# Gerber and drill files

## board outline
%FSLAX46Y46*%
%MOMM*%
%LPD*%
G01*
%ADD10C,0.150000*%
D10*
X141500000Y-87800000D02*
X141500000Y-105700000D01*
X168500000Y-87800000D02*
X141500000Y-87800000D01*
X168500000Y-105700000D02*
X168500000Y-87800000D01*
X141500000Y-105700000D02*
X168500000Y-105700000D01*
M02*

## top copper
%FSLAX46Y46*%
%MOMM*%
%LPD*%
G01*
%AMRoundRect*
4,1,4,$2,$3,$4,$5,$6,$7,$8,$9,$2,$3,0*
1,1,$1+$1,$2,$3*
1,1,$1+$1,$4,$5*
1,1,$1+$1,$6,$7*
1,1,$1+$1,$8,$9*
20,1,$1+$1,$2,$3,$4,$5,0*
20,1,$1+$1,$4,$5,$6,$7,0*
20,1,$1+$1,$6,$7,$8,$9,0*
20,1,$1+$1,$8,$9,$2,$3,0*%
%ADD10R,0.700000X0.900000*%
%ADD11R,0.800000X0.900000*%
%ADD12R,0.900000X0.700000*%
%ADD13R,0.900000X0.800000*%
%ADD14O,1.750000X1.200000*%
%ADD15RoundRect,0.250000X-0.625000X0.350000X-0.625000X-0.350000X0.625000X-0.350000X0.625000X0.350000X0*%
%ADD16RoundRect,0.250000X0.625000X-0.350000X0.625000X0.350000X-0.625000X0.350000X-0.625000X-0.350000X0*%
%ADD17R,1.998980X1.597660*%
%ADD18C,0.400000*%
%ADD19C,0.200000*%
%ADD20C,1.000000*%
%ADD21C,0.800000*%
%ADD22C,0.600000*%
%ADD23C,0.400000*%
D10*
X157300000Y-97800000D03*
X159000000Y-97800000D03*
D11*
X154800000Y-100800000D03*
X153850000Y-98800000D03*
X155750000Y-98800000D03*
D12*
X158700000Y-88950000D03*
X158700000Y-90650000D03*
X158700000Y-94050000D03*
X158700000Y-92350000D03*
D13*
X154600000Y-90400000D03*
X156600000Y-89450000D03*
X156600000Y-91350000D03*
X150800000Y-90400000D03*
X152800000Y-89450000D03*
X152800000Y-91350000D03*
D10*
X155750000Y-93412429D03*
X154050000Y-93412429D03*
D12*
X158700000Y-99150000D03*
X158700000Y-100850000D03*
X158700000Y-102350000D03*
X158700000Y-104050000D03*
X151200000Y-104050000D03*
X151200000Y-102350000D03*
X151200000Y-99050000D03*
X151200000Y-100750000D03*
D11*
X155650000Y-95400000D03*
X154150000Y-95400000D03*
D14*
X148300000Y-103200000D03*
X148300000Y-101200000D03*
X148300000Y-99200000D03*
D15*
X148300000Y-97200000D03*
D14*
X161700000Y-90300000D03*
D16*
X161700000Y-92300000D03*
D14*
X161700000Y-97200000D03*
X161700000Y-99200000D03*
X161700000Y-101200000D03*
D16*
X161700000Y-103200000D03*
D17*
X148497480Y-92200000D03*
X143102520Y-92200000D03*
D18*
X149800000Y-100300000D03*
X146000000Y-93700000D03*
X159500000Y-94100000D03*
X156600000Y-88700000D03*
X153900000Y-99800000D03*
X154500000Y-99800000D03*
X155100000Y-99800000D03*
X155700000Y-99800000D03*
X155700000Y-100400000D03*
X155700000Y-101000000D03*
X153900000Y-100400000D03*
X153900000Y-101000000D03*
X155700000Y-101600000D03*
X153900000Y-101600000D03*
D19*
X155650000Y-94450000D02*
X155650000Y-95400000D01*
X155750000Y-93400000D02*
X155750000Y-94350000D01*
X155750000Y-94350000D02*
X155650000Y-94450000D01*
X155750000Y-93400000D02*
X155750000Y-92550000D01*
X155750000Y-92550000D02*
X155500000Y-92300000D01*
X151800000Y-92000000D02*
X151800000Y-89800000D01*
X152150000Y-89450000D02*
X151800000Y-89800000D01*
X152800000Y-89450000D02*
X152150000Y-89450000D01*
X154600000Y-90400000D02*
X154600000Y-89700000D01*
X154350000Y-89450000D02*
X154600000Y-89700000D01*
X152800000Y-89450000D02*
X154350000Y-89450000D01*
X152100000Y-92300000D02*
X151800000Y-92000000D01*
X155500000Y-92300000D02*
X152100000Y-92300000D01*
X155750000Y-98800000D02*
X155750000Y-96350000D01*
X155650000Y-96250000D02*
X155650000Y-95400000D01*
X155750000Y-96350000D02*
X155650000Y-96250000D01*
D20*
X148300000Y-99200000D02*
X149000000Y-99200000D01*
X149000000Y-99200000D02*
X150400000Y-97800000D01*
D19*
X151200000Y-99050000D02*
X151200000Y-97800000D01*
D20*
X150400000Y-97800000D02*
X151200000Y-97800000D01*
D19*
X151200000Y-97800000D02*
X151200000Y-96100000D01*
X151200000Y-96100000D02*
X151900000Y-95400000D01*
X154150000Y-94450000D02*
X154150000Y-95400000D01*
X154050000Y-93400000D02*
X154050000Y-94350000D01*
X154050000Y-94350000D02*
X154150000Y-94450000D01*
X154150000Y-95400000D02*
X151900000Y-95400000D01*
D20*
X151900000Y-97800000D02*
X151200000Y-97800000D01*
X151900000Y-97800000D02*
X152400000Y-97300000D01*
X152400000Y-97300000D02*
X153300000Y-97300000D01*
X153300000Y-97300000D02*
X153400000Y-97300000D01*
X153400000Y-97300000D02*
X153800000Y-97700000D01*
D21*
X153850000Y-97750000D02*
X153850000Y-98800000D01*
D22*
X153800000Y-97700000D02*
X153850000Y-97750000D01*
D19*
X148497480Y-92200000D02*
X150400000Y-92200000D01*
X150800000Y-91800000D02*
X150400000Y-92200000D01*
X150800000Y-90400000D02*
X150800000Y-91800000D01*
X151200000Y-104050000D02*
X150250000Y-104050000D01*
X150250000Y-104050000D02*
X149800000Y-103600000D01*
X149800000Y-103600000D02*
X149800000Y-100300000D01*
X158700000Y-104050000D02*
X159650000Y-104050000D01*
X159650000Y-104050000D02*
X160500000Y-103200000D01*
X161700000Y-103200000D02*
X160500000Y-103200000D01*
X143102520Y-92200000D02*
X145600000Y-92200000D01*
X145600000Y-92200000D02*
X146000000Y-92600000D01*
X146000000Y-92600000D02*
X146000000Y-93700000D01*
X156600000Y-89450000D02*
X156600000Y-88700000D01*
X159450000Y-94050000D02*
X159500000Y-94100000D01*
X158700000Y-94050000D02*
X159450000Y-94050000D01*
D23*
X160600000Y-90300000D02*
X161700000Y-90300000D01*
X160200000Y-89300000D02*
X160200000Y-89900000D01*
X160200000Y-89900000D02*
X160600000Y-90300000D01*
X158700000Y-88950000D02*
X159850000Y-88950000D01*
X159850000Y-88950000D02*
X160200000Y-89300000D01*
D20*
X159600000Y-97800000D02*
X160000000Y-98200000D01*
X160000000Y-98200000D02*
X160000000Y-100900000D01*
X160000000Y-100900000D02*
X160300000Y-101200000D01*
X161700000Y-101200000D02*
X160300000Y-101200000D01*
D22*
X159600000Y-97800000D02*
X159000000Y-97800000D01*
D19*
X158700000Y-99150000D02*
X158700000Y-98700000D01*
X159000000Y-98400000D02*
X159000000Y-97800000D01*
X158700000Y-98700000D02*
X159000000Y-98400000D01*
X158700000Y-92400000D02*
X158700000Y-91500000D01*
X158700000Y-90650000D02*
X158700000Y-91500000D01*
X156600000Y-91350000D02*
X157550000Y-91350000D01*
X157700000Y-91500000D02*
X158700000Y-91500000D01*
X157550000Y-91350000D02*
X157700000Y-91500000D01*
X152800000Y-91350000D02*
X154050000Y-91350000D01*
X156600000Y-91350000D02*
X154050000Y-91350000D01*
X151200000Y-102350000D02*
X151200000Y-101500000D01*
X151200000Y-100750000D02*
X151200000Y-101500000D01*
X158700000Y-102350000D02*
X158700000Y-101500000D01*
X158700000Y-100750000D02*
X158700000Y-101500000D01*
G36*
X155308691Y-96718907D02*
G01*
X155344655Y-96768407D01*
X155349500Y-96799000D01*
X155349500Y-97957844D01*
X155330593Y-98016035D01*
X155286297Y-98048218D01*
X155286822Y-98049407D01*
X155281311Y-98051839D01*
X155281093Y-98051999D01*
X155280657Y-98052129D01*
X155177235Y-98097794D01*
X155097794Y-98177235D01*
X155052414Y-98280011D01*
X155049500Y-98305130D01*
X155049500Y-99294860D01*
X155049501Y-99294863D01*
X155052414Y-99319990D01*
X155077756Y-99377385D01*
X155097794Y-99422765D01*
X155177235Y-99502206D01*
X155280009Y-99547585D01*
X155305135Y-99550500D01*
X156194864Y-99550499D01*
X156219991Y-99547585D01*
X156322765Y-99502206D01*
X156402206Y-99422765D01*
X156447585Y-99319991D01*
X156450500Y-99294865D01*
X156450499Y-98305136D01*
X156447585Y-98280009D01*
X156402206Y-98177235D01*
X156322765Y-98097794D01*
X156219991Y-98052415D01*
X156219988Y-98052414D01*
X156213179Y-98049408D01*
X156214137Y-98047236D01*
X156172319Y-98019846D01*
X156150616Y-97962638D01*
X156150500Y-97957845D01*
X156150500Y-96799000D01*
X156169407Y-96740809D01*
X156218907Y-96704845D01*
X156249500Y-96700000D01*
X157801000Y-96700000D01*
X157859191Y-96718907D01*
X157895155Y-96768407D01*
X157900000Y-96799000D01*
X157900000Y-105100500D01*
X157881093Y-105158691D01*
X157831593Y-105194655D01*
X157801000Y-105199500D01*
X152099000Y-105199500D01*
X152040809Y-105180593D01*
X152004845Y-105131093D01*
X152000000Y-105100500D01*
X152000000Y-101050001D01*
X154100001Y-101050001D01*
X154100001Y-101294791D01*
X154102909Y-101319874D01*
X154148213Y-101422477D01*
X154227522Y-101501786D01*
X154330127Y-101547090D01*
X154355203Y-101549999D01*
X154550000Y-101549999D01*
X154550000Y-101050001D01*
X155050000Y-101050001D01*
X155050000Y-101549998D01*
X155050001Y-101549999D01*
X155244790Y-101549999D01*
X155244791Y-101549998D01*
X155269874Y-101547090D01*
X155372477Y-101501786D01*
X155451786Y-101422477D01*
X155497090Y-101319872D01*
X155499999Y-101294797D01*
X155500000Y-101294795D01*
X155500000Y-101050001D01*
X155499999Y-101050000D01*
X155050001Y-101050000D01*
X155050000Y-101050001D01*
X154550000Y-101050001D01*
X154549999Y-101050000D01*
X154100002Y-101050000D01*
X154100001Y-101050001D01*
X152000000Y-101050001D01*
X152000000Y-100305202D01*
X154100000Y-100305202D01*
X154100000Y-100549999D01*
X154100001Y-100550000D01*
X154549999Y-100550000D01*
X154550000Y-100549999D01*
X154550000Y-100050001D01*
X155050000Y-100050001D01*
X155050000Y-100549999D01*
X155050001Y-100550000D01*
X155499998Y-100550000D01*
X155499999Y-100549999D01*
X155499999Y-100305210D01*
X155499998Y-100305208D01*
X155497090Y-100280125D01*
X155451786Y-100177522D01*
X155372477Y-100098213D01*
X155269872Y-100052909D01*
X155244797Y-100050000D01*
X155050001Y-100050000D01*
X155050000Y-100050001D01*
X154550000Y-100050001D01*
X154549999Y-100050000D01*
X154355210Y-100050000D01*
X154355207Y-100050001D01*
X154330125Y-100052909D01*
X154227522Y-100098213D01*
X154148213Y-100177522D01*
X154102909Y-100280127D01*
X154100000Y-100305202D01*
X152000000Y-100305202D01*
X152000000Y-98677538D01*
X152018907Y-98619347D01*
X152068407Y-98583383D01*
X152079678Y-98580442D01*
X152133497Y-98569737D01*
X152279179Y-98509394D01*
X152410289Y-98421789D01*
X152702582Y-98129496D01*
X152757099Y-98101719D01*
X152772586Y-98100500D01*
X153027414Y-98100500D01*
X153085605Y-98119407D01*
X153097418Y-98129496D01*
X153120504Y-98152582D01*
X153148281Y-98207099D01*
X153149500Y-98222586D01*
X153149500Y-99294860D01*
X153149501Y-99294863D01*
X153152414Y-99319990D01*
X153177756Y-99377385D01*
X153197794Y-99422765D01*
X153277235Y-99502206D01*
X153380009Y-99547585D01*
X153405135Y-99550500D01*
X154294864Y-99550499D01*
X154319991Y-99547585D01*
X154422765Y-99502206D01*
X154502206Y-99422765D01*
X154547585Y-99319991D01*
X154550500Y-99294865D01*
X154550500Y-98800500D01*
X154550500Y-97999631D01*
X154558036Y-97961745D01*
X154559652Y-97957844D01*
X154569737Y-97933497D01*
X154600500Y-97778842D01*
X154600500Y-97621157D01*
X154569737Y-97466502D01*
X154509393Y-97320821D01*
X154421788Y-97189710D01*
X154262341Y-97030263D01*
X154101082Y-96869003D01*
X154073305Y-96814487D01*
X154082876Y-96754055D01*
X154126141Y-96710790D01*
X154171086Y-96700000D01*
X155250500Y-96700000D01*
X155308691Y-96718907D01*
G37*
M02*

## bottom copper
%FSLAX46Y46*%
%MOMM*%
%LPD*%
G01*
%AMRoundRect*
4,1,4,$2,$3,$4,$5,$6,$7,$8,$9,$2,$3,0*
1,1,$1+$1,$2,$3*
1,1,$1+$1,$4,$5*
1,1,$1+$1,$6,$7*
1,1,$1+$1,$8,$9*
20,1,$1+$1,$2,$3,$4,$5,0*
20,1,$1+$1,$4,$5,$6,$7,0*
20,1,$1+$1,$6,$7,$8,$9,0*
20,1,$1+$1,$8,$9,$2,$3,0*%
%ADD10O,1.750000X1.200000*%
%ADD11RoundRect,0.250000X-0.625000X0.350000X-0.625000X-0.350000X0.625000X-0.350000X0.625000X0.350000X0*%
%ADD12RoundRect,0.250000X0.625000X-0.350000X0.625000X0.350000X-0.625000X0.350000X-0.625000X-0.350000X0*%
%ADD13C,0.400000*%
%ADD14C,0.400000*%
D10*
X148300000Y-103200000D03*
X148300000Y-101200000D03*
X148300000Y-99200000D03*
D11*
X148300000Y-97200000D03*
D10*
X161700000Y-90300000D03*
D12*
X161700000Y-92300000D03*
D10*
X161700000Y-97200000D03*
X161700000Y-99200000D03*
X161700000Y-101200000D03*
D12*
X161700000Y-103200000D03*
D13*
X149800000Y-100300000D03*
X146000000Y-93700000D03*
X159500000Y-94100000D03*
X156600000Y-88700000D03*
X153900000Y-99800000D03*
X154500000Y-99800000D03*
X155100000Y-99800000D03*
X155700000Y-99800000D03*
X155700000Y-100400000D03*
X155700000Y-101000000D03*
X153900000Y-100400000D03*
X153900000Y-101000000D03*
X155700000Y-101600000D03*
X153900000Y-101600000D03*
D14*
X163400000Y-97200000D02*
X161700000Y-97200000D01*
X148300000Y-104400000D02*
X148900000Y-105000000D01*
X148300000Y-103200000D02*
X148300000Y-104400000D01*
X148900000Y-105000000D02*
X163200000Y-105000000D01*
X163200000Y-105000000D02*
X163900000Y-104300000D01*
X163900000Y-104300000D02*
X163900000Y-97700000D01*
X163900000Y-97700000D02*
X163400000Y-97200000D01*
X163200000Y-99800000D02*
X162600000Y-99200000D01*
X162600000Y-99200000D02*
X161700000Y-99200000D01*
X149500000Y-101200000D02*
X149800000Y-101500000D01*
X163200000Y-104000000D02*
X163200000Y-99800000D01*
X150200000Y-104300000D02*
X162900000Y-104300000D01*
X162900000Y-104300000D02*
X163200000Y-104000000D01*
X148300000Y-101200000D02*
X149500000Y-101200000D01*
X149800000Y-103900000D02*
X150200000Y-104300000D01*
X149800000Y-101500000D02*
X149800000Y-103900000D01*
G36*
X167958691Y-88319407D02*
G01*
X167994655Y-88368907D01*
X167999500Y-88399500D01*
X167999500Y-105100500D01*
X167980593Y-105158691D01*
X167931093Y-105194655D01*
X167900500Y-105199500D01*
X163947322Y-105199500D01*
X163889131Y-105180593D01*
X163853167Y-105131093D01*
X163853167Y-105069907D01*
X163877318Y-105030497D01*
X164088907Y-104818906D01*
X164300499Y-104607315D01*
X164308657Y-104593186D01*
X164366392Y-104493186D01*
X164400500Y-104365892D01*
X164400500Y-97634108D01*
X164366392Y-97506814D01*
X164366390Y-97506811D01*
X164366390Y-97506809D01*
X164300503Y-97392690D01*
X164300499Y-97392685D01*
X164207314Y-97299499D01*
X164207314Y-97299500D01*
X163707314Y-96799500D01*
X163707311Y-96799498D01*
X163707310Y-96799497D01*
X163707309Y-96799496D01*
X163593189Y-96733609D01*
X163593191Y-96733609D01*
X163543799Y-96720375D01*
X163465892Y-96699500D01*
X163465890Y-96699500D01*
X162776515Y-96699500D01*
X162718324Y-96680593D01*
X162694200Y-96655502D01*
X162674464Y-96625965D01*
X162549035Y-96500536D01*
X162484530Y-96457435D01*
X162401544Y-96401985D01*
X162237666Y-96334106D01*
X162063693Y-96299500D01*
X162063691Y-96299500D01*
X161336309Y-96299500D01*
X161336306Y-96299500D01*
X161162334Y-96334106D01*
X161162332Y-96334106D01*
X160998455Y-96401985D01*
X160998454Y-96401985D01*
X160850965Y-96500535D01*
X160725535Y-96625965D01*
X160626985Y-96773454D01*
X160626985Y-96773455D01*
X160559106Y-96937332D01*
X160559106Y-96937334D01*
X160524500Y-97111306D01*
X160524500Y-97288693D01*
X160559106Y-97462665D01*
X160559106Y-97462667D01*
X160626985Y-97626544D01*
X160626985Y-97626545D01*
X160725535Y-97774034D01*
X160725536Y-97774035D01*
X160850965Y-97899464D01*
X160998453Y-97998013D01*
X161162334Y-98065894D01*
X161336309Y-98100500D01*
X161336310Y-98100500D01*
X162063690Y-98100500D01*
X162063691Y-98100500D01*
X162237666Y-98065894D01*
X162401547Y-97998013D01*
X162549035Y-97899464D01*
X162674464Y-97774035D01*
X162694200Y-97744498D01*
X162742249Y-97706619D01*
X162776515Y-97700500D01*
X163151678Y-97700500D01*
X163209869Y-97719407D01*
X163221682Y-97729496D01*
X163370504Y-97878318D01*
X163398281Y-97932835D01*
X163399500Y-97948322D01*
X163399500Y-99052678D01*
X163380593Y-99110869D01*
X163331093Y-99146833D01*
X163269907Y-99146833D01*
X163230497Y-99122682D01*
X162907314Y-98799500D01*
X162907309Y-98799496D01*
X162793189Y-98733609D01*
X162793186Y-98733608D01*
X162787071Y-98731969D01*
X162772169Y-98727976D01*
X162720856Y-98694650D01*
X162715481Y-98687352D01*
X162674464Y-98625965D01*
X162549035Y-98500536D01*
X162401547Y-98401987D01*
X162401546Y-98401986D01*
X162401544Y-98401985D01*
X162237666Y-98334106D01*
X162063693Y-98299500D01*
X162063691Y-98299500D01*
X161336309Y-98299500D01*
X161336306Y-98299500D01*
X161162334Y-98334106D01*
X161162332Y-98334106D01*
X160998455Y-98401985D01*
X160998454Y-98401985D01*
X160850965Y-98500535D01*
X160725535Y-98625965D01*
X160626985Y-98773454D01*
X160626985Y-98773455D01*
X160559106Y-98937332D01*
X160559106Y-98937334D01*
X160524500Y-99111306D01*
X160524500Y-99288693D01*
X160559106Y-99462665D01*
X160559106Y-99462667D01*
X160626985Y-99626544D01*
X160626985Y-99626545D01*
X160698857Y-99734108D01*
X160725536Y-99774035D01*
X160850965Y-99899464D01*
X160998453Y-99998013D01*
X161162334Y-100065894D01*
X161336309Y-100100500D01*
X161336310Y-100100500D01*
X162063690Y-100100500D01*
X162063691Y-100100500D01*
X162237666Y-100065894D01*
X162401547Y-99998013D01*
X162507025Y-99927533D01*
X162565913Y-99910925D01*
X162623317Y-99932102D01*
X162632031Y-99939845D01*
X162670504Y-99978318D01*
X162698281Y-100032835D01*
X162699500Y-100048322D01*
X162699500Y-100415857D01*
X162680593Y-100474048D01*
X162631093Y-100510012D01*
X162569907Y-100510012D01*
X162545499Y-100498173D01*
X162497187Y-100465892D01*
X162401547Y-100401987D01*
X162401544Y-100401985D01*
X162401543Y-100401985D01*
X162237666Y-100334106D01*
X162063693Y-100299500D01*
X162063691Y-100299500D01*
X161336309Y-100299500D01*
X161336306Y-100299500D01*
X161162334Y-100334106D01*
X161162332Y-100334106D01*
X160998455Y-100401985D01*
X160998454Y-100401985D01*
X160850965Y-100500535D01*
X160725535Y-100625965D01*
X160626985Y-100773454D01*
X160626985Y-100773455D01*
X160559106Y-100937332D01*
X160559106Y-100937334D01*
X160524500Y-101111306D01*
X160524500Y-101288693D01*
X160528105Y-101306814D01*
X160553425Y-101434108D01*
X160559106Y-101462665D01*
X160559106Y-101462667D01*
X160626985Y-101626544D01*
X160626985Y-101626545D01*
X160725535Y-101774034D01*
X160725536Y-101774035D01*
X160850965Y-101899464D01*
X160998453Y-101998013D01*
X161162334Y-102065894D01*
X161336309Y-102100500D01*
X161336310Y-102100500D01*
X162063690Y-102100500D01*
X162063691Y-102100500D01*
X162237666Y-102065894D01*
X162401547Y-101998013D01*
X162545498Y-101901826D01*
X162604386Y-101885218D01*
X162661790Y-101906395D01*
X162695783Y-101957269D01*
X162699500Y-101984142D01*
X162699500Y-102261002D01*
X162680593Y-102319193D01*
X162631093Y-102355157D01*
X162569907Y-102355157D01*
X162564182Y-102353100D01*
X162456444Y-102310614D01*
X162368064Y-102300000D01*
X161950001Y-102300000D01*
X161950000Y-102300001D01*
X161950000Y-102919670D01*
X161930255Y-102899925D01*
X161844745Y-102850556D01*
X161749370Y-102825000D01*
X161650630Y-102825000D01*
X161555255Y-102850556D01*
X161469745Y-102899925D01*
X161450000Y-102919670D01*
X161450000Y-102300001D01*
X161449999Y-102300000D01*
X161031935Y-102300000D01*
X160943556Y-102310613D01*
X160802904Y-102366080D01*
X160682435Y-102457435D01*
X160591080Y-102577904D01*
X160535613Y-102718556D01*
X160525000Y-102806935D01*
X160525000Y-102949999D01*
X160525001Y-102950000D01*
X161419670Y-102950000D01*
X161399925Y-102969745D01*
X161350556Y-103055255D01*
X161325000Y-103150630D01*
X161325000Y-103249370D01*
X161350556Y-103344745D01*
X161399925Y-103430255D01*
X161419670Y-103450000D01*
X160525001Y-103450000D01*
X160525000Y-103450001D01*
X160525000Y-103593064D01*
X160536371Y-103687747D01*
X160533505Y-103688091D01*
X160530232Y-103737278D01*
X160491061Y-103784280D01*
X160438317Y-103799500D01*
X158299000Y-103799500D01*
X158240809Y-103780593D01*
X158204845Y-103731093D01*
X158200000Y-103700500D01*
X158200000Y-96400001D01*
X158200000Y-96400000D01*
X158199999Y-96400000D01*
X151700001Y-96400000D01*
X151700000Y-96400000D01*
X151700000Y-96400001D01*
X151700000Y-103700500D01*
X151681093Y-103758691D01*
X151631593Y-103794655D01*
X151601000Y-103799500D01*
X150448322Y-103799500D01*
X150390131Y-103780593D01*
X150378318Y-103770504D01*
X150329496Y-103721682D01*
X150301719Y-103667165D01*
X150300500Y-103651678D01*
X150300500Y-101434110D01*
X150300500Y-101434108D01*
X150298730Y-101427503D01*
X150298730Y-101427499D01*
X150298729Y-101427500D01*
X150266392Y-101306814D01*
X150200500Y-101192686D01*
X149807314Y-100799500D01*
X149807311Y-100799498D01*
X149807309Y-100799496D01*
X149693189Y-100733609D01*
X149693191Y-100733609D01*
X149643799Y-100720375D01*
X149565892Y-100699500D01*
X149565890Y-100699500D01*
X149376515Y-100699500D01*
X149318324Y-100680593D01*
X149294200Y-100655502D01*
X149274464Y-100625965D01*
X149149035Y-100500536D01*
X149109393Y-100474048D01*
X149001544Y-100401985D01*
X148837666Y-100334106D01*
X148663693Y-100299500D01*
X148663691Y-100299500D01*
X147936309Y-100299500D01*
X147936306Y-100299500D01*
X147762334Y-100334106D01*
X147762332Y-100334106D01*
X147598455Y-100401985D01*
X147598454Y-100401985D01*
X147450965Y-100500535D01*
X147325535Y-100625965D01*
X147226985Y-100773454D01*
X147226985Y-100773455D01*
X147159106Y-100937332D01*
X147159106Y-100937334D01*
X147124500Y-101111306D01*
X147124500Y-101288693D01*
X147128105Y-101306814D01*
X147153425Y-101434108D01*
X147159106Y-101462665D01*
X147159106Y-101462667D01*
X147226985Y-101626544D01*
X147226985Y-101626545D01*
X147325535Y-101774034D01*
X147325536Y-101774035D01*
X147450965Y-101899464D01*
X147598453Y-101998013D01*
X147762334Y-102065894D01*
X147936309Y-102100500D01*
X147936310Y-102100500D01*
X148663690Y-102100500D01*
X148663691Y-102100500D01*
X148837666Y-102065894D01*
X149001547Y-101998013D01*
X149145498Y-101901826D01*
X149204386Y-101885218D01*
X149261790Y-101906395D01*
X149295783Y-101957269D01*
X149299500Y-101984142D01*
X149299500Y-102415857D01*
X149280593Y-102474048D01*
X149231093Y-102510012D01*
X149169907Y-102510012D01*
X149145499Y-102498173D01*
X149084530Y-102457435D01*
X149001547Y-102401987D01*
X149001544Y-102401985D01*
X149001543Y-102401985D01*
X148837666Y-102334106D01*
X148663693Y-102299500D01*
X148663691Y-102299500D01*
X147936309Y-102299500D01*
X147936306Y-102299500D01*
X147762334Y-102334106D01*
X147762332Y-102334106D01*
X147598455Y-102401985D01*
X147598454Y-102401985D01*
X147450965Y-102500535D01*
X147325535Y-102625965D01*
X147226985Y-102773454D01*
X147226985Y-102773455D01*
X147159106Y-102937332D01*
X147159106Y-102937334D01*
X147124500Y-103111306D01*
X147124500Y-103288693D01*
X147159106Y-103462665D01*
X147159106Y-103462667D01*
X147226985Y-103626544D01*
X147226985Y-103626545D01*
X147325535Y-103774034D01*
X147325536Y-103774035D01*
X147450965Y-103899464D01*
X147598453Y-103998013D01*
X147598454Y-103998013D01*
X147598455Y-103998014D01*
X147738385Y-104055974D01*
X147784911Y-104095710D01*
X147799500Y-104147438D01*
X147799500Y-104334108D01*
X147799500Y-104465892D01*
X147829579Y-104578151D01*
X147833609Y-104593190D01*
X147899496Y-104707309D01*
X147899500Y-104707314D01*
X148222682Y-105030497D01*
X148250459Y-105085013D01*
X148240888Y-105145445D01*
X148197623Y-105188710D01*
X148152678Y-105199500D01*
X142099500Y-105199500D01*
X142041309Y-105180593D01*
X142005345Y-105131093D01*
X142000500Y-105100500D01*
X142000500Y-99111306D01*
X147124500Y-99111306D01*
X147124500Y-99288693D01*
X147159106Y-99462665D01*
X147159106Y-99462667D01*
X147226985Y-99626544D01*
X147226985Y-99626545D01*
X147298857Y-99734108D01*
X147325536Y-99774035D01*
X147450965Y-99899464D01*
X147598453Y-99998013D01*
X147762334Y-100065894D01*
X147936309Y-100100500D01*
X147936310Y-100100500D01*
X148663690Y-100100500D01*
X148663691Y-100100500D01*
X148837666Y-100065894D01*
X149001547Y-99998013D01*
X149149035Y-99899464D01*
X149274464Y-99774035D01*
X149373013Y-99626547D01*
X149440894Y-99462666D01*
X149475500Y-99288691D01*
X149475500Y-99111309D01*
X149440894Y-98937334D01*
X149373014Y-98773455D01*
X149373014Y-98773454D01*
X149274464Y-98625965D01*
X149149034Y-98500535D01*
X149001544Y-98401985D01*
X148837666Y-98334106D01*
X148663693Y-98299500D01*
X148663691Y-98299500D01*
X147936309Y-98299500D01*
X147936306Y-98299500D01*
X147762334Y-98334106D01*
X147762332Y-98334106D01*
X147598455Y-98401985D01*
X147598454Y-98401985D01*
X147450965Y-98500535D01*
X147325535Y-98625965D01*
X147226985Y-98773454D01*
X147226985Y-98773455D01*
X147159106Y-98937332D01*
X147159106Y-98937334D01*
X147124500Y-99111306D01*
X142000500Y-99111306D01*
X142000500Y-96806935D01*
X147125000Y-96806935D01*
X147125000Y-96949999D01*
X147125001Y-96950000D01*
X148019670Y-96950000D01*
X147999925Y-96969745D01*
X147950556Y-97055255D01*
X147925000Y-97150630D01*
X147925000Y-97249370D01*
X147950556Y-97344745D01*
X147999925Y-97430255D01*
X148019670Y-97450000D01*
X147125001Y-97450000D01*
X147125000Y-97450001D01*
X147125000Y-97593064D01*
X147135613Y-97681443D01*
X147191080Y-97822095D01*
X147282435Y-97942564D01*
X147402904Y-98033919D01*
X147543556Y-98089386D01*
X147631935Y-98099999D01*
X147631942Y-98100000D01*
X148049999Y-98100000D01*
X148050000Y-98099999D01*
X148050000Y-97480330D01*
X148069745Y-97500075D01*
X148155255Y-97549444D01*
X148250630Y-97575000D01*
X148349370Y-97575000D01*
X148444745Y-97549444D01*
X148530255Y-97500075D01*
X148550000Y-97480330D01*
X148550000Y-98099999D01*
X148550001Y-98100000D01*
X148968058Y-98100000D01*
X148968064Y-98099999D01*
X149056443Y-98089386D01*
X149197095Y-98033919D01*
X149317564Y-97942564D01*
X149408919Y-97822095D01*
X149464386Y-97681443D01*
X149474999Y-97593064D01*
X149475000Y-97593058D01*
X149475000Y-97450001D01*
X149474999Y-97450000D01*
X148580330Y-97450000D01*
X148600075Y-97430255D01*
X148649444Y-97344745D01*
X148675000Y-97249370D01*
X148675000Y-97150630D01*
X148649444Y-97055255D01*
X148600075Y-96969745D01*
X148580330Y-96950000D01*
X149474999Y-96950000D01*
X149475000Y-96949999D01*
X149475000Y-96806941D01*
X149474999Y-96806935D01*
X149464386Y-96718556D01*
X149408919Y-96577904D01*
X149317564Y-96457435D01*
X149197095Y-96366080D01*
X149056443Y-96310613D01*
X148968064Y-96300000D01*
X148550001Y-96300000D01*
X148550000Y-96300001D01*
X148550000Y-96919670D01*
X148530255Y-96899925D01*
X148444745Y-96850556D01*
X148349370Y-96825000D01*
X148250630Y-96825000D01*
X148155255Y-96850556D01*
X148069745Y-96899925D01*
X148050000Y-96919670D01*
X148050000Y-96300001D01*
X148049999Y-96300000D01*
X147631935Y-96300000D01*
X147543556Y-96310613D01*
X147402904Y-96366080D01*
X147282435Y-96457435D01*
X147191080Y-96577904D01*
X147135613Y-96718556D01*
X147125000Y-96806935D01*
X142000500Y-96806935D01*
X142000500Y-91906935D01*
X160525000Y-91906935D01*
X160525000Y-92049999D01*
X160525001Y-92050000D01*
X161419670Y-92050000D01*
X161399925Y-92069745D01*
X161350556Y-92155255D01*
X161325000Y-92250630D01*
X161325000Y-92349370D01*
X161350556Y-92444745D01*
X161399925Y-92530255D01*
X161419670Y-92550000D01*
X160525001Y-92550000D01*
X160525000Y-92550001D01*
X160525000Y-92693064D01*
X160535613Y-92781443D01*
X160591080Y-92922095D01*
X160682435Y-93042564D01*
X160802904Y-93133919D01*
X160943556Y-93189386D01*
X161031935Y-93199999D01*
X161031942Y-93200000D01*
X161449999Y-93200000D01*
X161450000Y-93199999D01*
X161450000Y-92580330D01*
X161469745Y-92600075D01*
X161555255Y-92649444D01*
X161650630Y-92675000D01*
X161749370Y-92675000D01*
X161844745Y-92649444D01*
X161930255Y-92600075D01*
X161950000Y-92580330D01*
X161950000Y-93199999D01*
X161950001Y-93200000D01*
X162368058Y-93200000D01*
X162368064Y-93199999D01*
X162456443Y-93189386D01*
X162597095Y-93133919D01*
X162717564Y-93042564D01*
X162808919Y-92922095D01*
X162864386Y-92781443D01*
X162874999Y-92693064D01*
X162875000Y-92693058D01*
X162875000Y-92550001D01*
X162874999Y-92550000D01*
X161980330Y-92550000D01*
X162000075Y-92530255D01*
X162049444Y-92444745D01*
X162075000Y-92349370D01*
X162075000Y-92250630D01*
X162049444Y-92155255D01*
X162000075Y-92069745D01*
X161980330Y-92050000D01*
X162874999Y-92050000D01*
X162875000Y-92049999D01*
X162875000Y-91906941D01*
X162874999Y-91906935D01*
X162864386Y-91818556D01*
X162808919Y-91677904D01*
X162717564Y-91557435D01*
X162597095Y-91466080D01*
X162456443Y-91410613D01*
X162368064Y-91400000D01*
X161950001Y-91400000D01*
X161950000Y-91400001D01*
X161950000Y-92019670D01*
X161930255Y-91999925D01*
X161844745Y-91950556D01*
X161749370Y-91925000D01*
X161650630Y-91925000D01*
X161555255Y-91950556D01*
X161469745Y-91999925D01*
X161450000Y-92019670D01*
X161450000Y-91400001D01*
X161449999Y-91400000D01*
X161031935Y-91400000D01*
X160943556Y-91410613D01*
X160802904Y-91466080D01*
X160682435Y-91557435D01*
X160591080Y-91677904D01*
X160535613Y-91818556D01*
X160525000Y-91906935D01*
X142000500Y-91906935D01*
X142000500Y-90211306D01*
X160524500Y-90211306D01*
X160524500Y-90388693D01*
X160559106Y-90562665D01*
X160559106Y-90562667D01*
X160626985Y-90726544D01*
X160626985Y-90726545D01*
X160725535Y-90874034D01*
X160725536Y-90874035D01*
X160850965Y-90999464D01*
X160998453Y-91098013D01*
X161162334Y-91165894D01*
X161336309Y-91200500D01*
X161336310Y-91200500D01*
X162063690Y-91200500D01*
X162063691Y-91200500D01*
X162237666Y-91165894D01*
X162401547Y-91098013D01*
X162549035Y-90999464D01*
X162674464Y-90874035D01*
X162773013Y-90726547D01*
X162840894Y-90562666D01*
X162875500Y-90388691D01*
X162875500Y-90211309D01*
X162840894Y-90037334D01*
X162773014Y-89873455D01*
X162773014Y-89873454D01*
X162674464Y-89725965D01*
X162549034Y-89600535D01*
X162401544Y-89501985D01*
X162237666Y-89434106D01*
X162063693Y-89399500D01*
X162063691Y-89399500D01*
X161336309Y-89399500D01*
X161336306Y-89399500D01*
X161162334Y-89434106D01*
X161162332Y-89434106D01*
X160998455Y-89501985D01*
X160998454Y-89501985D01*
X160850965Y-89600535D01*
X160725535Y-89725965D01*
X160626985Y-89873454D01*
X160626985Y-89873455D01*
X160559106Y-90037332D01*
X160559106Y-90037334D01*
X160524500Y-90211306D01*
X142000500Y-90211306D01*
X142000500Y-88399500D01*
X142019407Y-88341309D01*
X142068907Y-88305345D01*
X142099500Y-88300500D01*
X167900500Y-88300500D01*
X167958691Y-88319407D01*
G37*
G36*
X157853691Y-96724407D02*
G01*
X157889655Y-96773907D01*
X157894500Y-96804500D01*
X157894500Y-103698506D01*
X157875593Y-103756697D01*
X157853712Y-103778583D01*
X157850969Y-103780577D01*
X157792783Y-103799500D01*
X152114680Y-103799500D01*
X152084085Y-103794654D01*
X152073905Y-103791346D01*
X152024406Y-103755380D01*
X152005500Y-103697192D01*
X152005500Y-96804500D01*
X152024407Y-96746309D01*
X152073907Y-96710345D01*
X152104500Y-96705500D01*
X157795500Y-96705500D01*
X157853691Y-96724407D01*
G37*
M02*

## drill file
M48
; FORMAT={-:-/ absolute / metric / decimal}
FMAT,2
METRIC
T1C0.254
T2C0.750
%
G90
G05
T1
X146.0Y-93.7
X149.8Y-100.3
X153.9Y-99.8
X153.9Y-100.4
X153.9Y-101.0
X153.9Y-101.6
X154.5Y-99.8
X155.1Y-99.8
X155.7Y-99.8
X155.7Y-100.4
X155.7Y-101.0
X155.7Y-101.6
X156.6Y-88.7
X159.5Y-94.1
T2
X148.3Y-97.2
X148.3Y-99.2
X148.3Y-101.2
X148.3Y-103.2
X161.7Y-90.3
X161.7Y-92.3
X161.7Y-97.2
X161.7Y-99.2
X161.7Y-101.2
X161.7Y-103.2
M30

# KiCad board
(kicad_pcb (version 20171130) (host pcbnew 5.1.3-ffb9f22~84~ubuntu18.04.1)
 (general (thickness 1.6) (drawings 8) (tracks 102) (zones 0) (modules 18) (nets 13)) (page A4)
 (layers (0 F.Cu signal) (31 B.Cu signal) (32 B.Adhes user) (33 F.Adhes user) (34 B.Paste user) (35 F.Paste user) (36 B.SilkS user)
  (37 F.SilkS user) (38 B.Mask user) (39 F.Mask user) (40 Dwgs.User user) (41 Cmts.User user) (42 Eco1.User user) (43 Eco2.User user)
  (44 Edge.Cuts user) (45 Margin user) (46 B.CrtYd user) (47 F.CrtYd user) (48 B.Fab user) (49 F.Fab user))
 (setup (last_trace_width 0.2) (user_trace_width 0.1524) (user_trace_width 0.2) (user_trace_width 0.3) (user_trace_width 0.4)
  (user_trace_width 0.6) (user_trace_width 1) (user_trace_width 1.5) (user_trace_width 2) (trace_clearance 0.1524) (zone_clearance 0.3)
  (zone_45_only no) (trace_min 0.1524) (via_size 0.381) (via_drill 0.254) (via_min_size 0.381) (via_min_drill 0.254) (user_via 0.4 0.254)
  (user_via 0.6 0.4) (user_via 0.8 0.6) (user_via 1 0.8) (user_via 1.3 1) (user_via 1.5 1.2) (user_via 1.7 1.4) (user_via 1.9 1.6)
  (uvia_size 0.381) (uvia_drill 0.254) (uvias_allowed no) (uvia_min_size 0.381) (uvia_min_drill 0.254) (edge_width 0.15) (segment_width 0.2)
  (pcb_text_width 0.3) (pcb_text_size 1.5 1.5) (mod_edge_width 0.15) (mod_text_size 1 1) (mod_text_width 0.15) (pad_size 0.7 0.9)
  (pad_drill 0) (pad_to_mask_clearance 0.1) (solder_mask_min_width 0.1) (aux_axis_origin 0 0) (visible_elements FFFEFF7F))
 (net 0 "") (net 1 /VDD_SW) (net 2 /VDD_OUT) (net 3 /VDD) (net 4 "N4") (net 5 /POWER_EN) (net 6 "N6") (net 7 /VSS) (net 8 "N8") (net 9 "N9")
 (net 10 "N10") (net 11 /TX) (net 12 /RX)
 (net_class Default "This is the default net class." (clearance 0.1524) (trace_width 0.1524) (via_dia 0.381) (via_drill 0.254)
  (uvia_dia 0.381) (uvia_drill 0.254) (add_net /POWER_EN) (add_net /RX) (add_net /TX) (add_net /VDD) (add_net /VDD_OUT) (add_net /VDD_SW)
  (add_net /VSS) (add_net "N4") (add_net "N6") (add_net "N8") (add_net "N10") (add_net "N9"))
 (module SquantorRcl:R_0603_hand (layer F.Cu) (at 158.15 97.8 180)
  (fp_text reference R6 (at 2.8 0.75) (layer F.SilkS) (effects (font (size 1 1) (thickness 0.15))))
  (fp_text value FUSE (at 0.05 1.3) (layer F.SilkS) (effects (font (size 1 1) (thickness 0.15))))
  (pad 2 smd rect (at 0.85 0 180) (size 0.7 0.9) (layers F.Cu F.Paste F.Mask) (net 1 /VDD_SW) (zone_connect 2))
  (pad 1 smd rect (at -0.85 0 180) (size 0.7 0.9) (layers F.Cu F.Paste F.Mask) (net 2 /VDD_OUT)))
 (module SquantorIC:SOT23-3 (layer F.Cu) (at 154.8 99.8 180)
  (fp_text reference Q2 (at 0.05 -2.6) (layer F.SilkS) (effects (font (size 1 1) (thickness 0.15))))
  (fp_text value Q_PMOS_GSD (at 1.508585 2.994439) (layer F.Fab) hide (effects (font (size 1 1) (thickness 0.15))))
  (pad 3 smd rect (at 0 -1 180) (size 0.8 0.9) (layers F.Cu F.Paste F.Mask) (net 1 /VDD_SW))
  (pad 2 smd rect (at 0.95 1 180) (size 0.8 0.9) (layers F.Cu F.Paste F.Mask) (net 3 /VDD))
  (pad 1 smd rect (at -0.95 1 180) (size 0.8 0.9) (layers F.Cu F.Paste F.Mask) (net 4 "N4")))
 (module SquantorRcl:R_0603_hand (layer F.Cu) (at 158.7 89.8 90)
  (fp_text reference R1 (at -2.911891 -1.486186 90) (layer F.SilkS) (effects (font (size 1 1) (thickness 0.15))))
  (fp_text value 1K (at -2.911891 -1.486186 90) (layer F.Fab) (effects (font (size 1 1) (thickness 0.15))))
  (pad 2 smd rect (at 0.85 0 90) (size 0.7 0.9) (layers F.Cu F.Paste F.Mask) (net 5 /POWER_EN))
  (pad 1 smd rect (at -0.85 0 90) (size 0.7 0.9) (layers F.Cu F.Paste F.Mask) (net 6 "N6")))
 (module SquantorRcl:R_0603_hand (layer F.Cu) (at 158.7 93.2 270)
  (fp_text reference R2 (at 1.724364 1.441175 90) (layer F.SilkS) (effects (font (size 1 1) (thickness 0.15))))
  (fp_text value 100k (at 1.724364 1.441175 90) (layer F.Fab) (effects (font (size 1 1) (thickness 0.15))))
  (pad 2 smd rect (at 0.85 0 270) (size 0.7 0.9) (layers F.Cu F.Paste F.Mask) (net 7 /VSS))
  (pad 1 smd rect (at -0.85 0 270) (size 0.7 0.9) (layers F.Cu F.Paste F.Mask) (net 6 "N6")))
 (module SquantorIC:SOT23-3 (layer F.Cu) (at 155.6 90.4 90)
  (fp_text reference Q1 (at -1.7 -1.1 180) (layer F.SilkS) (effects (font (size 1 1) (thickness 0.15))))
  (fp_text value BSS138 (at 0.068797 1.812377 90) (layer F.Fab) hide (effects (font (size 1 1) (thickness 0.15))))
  (pad 3 smd rect (at 0 -1 90) (size 0.8 0.9) (layers F.Cu F.Paste F.Mask) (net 4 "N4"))
  (pad 2 smd rect (at 0.95 1 90) (size 0.8 0.9) (layers F.Cu F.Paste F.Mask) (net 7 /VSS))
  (pad 1 smd rect (at -0.95 1 90) (size 0.8 0.9) (layers F.Cu F.Paste F.Mask) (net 6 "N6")))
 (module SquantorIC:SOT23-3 (layer F.Cu) (at 151.8 90.4 90)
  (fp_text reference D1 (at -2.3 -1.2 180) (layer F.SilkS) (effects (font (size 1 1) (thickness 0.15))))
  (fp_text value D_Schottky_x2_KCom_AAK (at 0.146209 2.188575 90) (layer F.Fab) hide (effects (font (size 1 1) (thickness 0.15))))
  (pad 3 smd rect (at 0 -1 90) (size 0.8 0.9) (layers F.Cu F.Paste F.Mask) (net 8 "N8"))
  (pad 2 smd rect (at 0.95 1 90) (size 0.8 0.9) (layers F.Cu F.Paste F.Mask) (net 4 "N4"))
  (pad 1 smd rect (at -0.95 1 90) (size 0.8 0.9) (layers F.Cu F.Paste F.Mask) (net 6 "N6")))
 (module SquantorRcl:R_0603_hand (layer F.Cu) (at 154.9 93.412429)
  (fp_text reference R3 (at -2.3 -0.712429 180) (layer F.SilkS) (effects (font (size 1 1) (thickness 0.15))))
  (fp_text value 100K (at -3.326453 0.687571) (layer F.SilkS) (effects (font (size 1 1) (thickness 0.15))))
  (pad 2 smd rect (at 0.85 0) (size 0.7 0.9) (layers F.Cu F.Paste F.Mask) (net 4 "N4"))
  (pad 1 smd rect (at -0.85 0) (size 0.7 0.9) (layers F.Cu F.Paste F.Mask) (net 3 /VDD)))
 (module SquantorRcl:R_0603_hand (layer F.Cu) (at 158.7 100 90)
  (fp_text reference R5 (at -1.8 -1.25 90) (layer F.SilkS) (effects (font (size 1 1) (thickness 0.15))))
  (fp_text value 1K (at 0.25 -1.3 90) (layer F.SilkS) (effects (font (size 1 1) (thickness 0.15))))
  (pad 2 smd rect (at 0.85 0 90) (size 0.7 0.9) (layers F.Cu F.Paste F.Mask) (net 2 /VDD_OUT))
  (pad 1 smd rect (at -0.85 0 90) (size 0.7 0.9) (layers F.Cu F.Paste F.Mask) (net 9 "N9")))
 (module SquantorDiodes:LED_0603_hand (layer F.Cu) (at 158.7 103.2 90)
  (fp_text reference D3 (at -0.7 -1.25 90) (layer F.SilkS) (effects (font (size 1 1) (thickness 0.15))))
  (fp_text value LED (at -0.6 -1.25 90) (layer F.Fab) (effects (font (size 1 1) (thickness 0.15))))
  (pad 2 smd rect (at 0.85 0 90) (size 0.7 0.9) (layers F.Cu F.Paste F.Mask) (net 9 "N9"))
  (pad 1 smd rect (at -0.85 0 90) (size 0.7 0.9) (layers F.Cu F.Paste F.Mask) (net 7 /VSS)))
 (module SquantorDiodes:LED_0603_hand (layer F.Cu) (at 151.2 103.2 90)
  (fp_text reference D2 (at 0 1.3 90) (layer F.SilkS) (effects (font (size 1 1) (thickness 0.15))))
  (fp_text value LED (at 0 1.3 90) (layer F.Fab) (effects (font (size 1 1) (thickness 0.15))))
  (pad 1 smd rect (at -0.85 0 90) (size 0.7 0.9) (layers F.Cu F.Paste F.Mask) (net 7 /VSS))
  (pad 2 smd rect (at 0.85 0 90) (size 0.7 0.9) (layers F.Cu F.Paste F.Mask) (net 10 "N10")))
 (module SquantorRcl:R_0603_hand (layer F.Cu) (at 151.2 99.9 90)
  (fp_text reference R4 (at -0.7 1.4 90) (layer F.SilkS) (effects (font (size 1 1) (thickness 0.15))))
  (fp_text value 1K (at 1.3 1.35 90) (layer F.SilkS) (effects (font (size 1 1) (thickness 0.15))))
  (pad 2 smd rect (at 0.85 0 90) (size 0.7 0.9) (layers F.Cu F.Paste F.Mask) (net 3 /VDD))
  (pad 1 smd rect (at -0.85 0 90) (size 0.7 0.9) (layers F.Cu F.Paste F.Mask) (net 10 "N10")))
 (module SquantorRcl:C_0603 (layer F.Cu) (at 154.9 95.4)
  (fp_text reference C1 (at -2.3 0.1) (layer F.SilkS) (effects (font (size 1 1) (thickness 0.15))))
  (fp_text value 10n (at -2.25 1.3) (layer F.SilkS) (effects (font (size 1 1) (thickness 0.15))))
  (pad 2 smd rect (at 0.75 0) (size 0.8 0.9) (layers F.Cu F.Paste F.Mask) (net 4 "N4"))
  (pad 1 smd rect (at -0.75 0) (size 0.8 0.9) (layers F.Cu F.Paste F.Mask) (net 3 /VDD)))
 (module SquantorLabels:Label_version (layer B.Cu) (at 153.4 95.4 180)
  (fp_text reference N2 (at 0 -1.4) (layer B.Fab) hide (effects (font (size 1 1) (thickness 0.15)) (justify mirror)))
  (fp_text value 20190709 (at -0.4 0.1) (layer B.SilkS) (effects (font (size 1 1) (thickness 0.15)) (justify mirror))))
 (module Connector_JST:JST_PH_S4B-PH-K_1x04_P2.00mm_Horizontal (layer F.Cu) (at 148.3 97.2 270)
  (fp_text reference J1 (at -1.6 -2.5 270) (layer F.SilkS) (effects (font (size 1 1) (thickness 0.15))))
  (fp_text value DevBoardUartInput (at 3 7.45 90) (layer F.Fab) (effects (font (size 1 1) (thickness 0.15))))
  (pad 4 thru_hole oval (at 6 0 270) (size 1.2 1.75) (drill 0.75) (layers *.Cu *.Mask) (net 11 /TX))
  (pad 3 thru_hole oval (at 4 0 270) (size 1.2 1.75) (drill 0.75) (layers *.Cu *.Mask) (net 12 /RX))
  (pad 2 thru_hole oval (at 2 0 270) (size 1.2 1.75) (drill 0.75) (layers *.Cu *.Mask) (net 3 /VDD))
  (pad 1 thru_hole roundrect (at 0 0 270) (size 1.2 1.75) (drill 0.75) (layers *.Cu *.Mask) (roundrect_rratio 0.208333) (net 7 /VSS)))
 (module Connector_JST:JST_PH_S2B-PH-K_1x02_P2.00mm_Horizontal (layer F.Cu) (at 161.7 92.3 90)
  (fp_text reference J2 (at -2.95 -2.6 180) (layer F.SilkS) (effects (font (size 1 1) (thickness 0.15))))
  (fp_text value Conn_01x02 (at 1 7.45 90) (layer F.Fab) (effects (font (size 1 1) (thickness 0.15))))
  (pad 2 thru_hole oval (at 2 0 90) (size 1.2 1.75) (drill 0.75) (layers *.Cu *.Mask) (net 5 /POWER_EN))
  (pad 1 thru_hole roundrect (at 0 0 90) (size 1.2 1.75) (drill 0.75) (layers *.Cu *.Mask) (roundrect_rratio 0.208333) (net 7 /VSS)))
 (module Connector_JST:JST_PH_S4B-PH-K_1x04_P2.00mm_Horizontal (layer F.Cu) (at 161.7 103.2 90)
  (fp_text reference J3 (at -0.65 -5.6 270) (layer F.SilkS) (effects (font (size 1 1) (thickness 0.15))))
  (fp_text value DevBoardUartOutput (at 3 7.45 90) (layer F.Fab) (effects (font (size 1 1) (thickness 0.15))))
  (pad 4 thru_hole oval (at 6 0 90) (size 1.2 1.75) (drill 0.75) (layers *.Cu *.Mask) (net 11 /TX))
  (pad 3 thru_hole oval (at 4 0 90) (size 1.2 1.75) (drill 0.75) (layers *.Cu *.Mask) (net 12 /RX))
  (pad 2 thru_hole oval (at 2 0 90) (size 1.2 1.75) (drill 0.75) (layers *.Cu *.Mask) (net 2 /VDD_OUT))
  (pad 1 thru_hole roundrect (at 0 0 90) (size 1.2 1.75) (drill 0.75) (layers *.Cu *.Mask) (roundrect_rratio 0.208333) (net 7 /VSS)))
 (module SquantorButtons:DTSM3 (layer F.Cu) (at 145.8 92.2)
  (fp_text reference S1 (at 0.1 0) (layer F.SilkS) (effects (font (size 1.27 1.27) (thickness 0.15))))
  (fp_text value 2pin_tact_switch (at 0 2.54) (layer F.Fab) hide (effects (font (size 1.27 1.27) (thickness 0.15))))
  (pad 2 smd rect (at 2.69748 0) (size 1.99898 1.59766) (layers F.Cu F.Paste F.Mask) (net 8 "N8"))
  (pad 1 smd rect (at -2.69748 0) (size 1.99898 1.59766) (layers F.Cu F.Paste F.Mask) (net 7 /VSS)))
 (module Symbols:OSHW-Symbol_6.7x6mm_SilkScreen (layer B.Cu) (at 154.5 91.5 180)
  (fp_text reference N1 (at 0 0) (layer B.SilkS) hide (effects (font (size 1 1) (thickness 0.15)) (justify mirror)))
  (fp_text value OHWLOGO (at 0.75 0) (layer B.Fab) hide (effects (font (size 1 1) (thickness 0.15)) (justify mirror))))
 (gr_line (start 141.5 87.8) (end 141.5 105.7) (layer Edge.Cuts) (width 0.15))
 (gr_line (start 168.5 87.8) (end 141.5 87.8) (layer Edge.Cuts) (width 0.15))
 (gr_line (start 168.5 105.7) (end 168.5 87.8) (layer Edge.Cuts) (width 0.15))
 (gr_line (start 141.5 105.7) (end 168.5 105.7) (layer Edge.Cuts) (width 0.15))
 (segment (start 155.65 94.45) (end 155.65 95.4) (width 0.2) (layer F.Cu) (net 4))
 (segment (start 155.75 93.4) (end 155.75 94.35) (width 0.2) (layer F.Cu) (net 4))
 (segment (start 155.75 94.35) (end 155.65 94.45) (width 0.2) (layer F.Cu) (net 4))
 (segment (start 155.75 93.4) (end 155.75 92.55) (width 0.2) (layer F.Cu) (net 4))
 (segment (start 155.75 92.55) (end 155.5 92.3) (width 0.2) (layer F.Cu) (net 4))
 (segment (start 151.8 92) (end 151.8 89.8) (width 0.2) (layer F.Cu) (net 4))
 (segment (start 152.15 89.45) (end 151.8 89.8) (width 0.2) (layer F.Cu) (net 4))
 (segment (start 152.8 89.45) (end 152.15 89.45) (width 0.2) (layer F.Cu) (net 4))
 (segment (start 154.6 90.4) (end 154.6 89.7) (width 0.2) (layer F.Cu) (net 4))
 (segment (start 154.35 89.45) (end 154.6 89.7) (width 0.2) (layer F.Cu) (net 4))
 (segment (start 152.8 89.45) (end 154.35 89.45) (width 0.2) (layer F.Cu) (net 4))
 (segment (start 152.1 92.3) (end 151.8 92) (width 0.2) (layer F.Cu) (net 4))
 (segment (start 155.5 92.3) (end 152.1 92.3) (width 0.2) (layer F.Cu) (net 4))
 (segment (start 155.75 98.8) (end 155.75 96.35) (width 0.2) (layer F.Cu) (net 4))
 (segment (start 155.65 96.25) (end 155.65 95.4) (width 0.2) (layer F.Cu) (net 4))
 (segment (start 155.75 96.35) (end 155.65 96.25) (width 0.2) (layer F.Cu) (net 4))
 (segment (start 148.3 99.2) (end 149 99.2) (width 1) (layer F.Cu) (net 3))
 (segment (start 149 99.2) (end 150.4 97.8) (width 1) (layer F.Cu) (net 3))
 (segment (start 151.2 99.05) (end 151.2 97.8) (width 0.2) (layer F.Cu) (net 3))
 (segment (start 150.4 97.8) (end 151.2 97.8) (width 1) (layer F.Cu) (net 3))
 (segment (start 151.2 97.8) (end 151.2 96.1) (width 0.2) (layer F.Cu) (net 3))
 (segment (start 151.2 96.1) (end 151.9 95.4) (width 0.2) (layer F.Cu) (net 3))
 (segment (start 154.15 94.45) (end 154.15 95.4) (width 0.2) (layer F.Cu) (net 3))
 (segment (start 154.05 93.4) (end 154.05 94.35) (width 0.2) (layer F.Cu) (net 3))
 (segment (start 154.05 94.35) (end 154.15 94.45) (width 0.2) (layer F.Cu) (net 3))
 (segment (start 154.15 95.4) (end 151.9 95.4) (width 0.2) (layer F.Cu) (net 3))
 (segment (start 151.9 97.8) (end 151.2 97.8) (width 1) (layer F.Cu) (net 3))
 (segment (start 151.9 97.8) (end 152.4 97.3) (width 1) (layer F.Cu) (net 3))
 (segment (start 152.4 97.3) (end 153.3 97.3) (width 1) (layer F.Cu) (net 3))
 (segment (start 153.3 97.3) (end 153.4 97.3) (width 1) (layer F.Cu) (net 3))
 (segment (start 153.4 97.3) (end 153.8 97.7) (width 1) (layer F.Cu) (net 3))
 (segment (start 153.85 97.75) (end 153.85 98.8) (width 0.8) (layer F.Cu) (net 3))
 (segment (start 153.8 97.7) (end 153.85 97.75) (width 0.6) (layer F.Cu) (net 3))
 (segment (start 148.49748 92.2) (end 150.4 92.2) (width 0.2) (layer F.Cu) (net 8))
 (segment (start 150.8 91.8) (end 150.4 92.2) (width 0.2) (layer F.Cu) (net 8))
 (segment (start 150.8 90.4) (end 150.8 91.8) (width 0.2) (layer F.Cu) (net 8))
 (segment (start 163.4 97.2) (end 161.7 97.2) (width 0.4) (layer B.Cu) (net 11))
 (segment (start 148.3 104.4) (end 148.9 105) (width 0.4) (layer B.Cu) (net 11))
 (segment (start 148.3 103.2) (end 148.3 104.4) (width 0.4) (layer B.Cu) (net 11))
 (segment (start 148.9 105) (end 163.2 105) (width 0.4) (layer B.Cu) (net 11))
 (segment (start 163.2 105) (end 163.9 104.3) (width 0.4) (layer B.Cu) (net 11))
 (segment (start 163.9 104.3) (end 163.9 97.7) (width 0.4) (layer B.Cu) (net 11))
 (segment (start 163.9 97.7) (end 163.4 97.2) (width 0.4) (layer B.Cu) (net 11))
 (segment (start 163.2 99.8) (end 162.6 99.2) (width 0.4) (layer B.Cu) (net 12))
 (segment (start 162.6 99.2) (end 161.7 99.2) (width 0.4) (layer B.Cu) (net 12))
 (segment (start 149.5 101.2) (end 149.8 101.5) (width 0.4) (layer B.Cu) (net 12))
 (segment (start 163.2 104) (end 163.2 99.8) (width 0.4) (layer B.Cu) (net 12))
 (segment (start 150.2 104.3) (end 162.9 104.3) (width 0.4) (layer B.Cu) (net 12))
 (segment (start 162.9 104.3) (end 163.2 104) (width 0.4) (layer B.Cu) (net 12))
 (segment (start 148.3 101.2) (end 149.5 101.2) (width 0.4) (layer B.Cu) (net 12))
 (segment (start 149.8 103.9) (end 150.2 104.3) (width 0.4) (layer B.Cu) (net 12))
 (segment (start 149.8 101.5) (end 149.8 103.9) (width 0.4) (layer B.Cu) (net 12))
 (segment (start 151.2 104.05) (end 150.25 104.05) (width 0.2) (layer F.Cu) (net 7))
 (segment (start 150.25 104.05) (end 149.8 103.6) (width 0.2) (layer F.Cu) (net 7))
 (via (at 149.8 100.3) (size 0.4) (drill 0.254) (layers F.Cu B.Cu) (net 7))
 (segment (start 149.8 103.6) (end 149.8 100.3) (width 0.2) (layer F.Cu) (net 7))
 (segment (start 158.7 104.05) (end 159.65 104.05) (width 0.2) (layer F.Cu) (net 7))
 (segment (start 159.65 104.05) (end 160.5 103.2) (width 0.2) (layer F.Cu) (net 7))
 (segment (start 161.7 103.2) (end 160.5 103.2) (width 0.2) (layer F.Cu) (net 7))
 (segment (start 143.10252 92.2) (end 145.6 92.2) (width 0.2) (layer F.Cu) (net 7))
 (via (at 146 93.7) (size 0.4) (drill 0.254) (layers F.Cu B.Cu) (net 7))
 (segment (start 145.6 92.2) (end 146 92.6) (width 0.2) (layer F.Cu) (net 7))
 (segment (start 146 92.6) (end 146 93.7) (width 0.2) (layer F.Cu) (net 7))
 (via (at 159.5 94.1) (size 0.4) (drill 0.254) (layers F.Cu B.Cu) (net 7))
 (via (at 156.6 88.7) (size 0.4) (drill 0.254) (layers F.Cu B.Cu) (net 7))
 (segment (start 156.6 89.45) (end 156.6 88.7) (width 0.2) (layer F.Cu) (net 7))
 (segment (start 159.45 94.05) (end 159.5 94.1) (width 0.2) (layer F.Cu) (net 7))
 (segment (start 158.7 94.05) (end 159.45 94.05) (width 0.2) (layer F.Cu) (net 7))
 (segment (start 160.6 90.3) (end 161.7 90.3) (width 0.4) (layer F.Cu) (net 5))
 (segment (start 160.2 89.3) (end 160.2 89.9) (width 0.4) (layer F.Cu) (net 5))
 (segment (start 160.2 89.9) (end 160.6 90.3) (width 0.4) (layer F.Cu) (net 5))
 (segment (start 158.7 88.95) (end 159.85 88.95) (width 0.4) (layer F.Cu) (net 5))
 (segment (start 159.85 88.95) (end 160.2 89.3) (width 0.4) (layer F.Cu) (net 5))
 (via (at 153.9 99.8) (size 0.4) (drill 0.254) (layers F.Cu B.Cu) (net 1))
 (via (at 154.5 99.8) (size 0.4) (drill 0.254) (layers F.Cu B.Cu) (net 1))
 (via (at 155.1 99.8) (size 0.4) (drill 0.254) (layers F.Cu B.Cu) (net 1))
 (via (at 155.7 99.8) (size 0.4) (drill 0.254) (layers F.Cu B.Cu) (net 1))
 (via (at 155.7 100.4) (size 0.4) (drill 0.254) (layers F.Cu B.Cu) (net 1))
 (via (at 155.7 101) (size 0.4) (drill 0.254) (layers F.Cu B.Cu) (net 1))
 (via (at 153.9 100.4) (size 0.4) (drill 0.254) (layers F.Cu B.Cu) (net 1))
 (via (at 153.9 101) (size 0.4) (drill 0.254) (layers F.Cu B.Cu) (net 1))
 (via (at 155.7 101.6) (size 0.4) (drill 0.254) (layers F.Cu B.Cu) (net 1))
 (via (at 153.9 101.6) (size 0.4) (drill 0.254) (layers F.Cu B.Cu) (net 1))
 (segment (start 159.6 97.8) (end 160 98.2) (width 1) (layer F.Cu) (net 2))
 (segment (start 160 98.2) (end 160 100.9) (width 1) (layer F.Cu) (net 2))
 (segment (start 160 100.9) (end 160.3 101.2) (width 1) (layer F.Cu) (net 2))
 (segment (start 161.7 101.2) (end 160.3 101.2) (width 1) (layer F.Cu) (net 2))
 (segment (start 159.6 97.8) (end 159 97.8) (width 0.6) (layer F.Cu) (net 2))
 (segment (start 158.7 99.15) (end 158.7 98.7) (width 0.2) (layer F.Cu) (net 2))
 (segment (start 159 98.4) (end 159 97.8) (width 0.2) (layer F.Cu) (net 2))
 (segment (start 158.7 98.7) (end 159 98.4) (width 0.2) (layer F.Cu) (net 2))
 (segment (start 158.7 92.4) (end 158.7 91.5) (width 0.2) (layer F.Cu) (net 6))
 (segment (start 158.7 90.65) (end 158.7 91.5) (width 0.2) (layer F.Cu) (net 6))
 (segment (start 156.6 91.35) (end 157.55 91.35) (width 0.2) (layer F.Cu) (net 6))
 (segment (start 157.7 91.5) (end 158.7 91.5) (width 0.2) (layer F.Cu) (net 6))
 (segment (start 157.55 91.35) (end 157.7 91.5) (width 0.2) (layer F.Cu) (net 6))
 (segment (start 152.8 91.35) (end 154.05 91.35) (width 0.2) (layer F.Cu) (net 6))
 (segment (start 156.6 91.35) (end 154.05 91.35) (width 0.2) (layer F.Cu) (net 6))
 (segment (start 151.2 102.35) (end 151.2 101.5) (width 0.2) (layer F.Cu) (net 10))
 (segment (start 151.2 100.75) (end 151.2 101.5) (width 0.2) (layer F.Cu) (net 10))
 (segment (start 158.7 102.35) (end 158.7 101.5) (width 0.2) (layer F.Cu) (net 9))
 (segment (start 158.7 100.75) (end 158.7 101.5) (width 0.2) (layer F.Cu) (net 9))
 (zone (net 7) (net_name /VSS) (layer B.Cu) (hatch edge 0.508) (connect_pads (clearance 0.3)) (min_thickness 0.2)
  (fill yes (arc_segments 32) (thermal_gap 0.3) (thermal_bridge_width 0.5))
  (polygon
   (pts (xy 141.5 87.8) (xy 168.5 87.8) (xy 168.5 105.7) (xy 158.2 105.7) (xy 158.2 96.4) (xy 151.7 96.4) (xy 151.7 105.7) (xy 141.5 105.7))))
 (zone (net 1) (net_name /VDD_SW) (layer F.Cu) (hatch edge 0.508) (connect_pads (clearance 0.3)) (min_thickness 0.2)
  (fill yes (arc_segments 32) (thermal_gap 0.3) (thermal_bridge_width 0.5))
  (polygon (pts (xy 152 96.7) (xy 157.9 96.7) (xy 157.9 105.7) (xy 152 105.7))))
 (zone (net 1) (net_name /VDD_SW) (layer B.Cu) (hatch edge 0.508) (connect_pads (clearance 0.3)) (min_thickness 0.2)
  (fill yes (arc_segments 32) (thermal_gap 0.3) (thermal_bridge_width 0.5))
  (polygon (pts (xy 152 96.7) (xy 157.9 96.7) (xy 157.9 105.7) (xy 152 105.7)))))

